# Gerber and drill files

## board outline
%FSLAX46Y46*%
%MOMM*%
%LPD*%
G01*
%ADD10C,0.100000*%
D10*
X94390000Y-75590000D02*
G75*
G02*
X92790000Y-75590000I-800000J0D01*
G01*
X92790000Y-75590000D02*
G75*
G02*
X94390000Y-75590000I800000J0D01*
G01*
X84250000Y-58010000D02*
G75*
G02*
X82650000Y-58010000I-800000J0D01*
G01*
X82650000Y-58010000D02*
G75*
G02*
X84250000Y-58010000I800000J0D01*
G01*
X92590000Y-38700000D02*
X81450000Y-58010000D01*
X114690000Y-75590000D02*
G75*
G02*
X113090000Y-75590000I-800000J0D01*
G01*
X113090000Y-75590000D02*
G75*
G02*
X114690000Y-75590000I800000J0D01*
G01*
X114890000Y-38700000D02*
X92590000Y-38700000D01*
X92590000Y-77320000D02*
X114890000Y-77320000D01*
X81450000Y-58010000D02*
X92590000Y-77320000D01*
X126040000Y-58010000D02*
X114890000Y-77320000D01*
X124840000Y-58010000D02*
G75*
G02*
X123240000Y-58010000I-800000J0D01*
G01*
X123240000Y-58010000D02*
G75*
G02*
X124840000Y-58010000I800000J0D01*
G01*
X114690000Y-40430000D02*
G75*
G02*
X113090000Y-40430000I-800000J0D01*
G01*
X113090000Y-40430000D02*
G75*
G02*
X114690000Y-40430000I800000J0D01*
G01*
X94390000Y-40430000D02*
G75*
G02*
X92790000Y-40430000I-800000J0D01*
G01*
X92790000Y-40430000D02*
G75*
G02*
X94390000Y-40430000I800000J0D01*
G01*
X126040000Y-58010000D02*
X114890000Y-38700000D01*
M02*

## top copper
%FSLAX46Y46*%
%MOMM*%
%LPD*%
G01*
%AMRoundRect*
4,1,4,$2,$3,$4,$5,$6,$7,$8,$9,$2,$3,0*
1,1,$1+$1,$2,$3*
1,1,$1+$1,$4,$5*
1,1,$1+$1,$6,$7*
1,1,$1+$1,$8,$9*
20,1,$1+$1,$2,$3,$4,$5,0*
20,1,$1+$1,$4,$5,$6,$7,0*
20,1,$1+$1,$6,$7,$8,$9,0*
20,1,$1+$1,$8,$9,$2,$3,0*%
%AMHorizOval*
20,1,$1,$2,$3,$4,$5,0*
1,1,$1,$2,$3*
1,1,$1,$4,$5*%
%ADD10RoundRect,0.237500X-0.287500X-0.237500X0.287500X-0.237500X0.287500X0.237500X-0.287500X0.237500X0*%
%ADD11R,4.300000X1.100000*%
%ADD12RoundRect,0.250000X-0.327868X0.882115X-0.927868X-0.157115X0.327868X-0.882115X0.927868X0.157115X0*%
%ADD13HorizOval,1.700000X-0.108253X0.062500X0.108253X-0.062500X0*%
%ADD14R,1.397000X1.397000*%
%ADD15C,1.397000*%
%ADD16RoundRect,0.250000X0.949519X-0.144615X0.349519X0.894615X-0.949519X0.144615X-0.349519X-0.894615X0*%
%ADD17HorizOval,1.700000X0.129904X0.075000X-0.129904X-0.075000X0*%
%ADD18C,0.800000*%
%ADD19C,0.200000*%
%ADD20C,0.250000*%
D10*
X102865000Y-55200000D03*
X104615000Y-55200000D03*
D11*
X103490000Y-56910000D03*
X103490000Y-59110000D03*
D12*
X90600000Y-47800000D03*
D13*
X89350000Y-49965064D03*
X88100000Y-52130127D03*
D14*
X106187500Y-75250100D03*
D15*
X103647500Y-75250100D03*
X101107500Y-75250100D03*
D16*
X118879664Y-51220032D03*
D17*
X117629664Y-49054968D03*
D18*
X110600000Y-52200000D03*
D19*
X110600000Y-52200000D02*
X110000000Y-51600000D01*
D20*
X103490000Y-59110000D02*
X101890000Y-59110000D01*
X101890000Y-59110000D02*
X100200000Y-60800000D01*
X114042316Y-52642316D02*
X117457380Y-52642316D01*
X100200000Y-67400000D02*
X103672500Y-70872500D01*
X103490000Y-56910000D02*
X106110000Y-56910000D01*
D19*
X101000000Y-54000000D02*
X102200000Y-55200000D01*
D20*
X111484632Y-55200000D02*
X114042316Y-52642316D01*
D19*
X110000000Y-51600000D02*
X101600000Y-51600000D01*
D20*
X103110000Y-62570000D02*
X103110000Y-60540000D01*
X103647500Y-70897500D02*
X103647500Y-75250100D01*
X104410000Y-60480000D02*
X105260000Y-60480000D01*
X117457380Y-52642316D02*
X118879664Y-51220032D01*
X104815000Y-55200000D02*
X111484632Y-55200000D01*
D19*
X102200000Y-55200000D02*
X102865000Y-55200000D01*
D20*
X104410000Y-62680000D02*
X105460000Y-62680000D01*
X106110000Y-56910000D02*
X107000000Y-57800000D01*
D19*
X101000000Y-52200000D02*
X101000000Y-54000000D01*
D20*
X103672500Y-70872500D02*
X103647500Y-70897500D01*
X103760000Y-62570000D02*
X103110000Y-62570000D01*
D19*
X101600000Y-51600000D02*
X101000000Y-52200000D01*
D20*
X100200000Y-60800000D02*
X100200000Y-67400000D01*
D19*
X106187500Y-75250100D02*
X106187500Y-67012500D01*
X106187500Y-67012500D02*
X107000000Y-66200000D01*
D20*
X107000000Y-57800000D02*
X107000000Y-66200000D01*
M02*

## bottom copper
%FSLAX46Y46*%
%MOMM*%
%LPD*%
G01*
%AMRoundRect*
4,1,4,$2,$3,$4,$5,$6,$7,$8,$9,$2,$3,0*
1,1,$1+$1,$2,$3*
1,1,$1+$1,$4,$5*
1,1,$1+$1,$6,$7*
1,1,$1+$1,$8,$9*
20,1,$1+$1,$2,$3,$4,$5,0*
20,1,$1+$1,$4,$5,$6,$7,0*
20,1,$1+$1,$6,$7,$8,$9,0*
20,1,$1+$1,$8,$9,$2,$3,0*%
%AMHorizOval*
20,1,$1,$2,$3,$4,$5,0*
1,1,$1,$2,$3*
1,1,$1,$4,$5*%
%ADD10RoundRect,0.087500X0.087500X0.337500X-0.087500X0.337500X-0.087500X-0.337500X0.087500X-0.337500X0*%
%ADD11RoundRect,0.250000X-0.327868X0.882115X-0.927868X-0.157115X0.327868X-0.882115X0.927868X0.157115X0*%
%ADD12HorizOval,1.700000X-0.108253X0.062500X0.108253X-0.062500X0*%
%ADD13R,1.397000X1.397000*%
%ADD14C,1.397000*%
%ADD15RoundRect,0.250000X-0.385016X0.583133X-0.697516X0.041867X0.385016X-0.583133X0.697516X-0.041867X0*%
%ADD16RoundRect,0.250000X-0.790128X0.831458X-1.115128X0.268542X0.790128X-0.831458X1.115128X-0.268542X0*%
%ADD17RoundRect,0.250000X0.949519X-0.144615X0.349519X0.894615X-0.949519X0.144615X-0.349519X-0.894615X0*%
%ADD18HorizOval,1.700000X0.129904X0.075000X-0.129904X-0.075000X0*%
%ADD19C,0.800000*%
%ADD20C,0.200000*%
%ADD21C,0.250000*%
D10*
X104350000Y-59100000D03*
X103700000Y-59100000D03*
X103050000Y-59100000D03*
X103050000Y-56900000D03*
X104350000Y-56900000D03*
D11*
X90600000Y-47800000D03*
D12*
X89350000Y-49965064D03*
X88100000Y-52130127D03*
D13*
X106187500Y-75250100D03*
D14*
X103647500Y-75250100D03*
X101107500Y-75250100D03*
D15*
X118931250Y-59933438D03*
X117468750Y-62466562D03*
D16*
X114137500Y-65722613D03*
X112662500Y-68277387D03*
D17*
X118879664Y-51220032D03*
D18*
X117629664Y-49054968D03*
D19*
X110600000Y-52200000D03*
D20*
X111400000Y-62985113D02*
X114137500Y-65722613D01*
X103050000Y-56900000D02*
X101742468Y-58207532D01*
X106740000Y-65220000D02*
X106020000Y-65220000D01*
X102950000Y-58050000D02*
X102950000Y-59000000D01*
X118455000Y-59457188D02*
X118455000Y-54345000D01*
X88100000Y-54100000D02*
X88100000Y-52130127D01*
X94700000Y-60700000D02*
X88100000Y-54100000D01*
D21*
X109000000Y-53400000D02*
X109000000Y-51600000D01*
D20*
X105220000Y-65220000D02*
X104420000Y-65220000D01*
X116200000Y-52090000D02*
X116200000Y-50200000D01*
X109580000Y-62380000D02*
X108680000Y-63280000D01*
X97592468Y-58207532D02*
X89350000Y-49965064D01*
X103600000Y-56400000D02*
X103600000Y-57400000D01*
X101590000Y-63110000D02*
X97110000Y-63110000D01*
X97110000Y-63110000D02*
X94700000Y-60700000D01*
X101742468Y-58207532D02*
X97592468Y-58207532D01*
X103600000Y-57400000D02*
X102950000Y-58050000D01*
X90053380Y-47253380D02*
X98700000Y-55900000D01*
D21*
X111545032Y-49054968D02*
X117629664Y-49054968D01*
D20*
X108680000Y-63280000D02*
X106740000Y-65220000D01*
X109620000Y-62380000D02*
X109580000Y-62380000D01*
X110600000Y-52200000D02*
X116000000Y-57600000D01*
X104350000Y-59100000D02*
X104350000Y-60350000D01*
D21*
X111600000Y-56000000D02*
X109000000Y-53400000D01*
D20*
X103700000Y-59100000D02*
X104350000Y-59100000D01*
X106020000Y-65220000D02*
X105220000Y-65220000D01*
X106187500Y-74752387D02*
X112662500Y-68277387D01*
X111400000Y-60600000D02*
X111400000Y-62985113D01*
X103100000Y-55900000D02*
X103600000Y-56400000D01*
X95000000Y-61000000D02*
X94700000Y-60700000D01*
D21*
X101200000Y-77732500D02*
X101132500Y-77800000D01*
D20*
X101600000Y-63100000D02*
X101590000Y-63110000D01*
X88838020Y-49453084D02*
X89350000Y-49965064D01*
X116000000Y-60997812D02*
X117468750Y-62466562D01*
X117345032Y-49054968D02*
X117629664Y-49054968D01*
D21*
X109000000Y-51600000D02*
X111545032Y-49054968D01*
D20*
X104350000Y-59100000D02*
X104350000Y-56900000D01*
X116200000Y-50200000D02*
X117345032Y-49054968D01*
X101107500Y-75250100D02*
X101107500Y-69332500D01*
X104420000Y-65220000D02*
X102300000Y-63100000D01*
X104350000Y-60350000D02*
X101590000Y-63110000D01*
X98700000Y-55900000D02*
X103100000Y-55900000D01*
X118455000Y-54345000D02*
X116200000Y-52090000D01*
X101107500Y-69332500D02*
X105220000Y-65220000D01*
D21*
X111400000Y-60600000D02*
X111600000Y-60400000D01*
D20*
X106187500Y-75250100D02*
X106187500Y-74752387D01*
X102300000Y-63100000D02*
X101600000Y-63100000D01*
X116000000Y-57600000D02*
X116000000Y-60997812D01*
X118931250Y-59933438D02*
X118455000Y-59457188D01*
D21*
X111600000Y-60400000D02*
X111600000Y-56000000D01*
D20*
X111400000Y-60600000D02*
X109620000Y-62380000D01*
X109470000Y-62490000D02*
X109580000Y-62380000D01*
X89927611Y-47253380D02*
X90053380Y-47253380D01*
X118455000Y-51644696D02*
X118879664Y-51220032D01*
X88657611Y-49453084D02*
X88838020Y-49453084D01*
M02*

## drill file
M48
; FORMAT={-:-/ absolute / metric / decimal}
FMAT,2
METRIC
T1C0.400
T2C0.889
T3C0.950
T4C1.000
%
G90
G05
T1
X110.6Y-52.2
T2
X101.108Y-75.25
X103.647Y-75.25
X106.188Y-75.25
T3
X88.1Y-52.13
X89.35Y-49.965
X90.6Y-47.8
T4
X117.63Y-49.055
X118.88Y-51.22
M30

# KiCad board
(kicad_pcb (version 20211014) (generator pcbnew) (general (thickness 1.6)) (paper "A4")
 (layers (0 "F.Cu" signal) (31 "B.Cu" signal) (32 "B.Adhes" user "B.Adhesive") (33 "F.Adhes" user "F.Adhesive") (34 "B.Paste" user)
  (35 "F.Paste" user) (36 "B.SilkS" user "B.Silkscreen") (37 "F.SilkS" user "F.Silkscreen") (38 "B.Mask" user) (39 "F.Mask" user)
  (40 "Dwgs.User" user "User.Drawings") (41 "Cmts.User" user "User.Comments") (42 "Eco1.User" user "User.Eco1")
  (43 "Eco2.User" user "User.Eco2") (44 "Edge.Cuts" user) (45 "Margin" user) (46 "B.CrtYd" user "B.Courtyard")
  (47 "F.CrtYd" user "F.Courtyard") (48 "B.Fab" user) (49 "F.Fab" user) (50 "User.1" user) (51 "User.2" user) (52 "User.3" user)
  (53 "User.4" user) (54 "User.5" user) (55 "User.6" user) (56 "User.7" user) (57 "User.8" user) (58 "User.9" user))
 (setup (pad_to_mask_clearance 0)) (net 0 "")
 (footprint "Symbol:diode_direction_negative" (layer "F.Cu") (at 103.8 52.65)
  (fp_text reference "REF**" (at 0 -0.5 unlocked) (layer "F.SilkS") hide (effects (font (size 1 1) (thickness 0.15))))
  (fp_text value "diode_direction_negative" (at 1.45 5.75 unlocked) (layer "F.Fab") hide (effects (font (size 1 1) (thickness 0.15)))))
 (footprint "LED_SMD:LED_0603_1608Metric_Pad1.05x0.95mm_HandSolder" (layer "F.Cu") (at 103.74 55.2)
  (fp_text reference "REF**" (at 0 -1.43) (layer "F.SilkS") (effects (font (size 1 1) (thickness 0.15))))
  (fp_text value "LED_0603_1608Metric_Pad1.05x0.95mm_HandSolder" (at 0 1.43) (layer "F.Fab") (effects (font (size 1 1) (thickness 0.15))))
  (pad "1" smd roundrect (at -0.875 0) (size 1.05 0.95) (layers "F.Cu" "F.Paste" "F.Mask") (roundrect_rratio 0.25))
  (pad "2" smd roundrect (at 0.875 0) (size 1.05 0.95) (layers "F.Cu" "F.Paste" "F.Mask") (roundrect_rratio 0.25)))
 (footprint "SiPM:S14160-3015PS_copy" (layer "F.Cu") (at 103.74 58.01)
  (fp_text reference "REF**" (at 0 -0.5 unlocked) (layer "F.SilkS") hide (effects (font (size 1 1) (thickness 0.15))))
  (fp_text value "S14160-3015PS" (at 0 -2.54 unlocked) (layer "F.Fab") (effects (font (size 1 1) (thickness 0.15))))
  (pad "1" smd rect (at -0.25 -1.1) (size 4.3 1.1) (layers "F.Cu" "F.Paste" "F.Mask"))
  (pad "2" smd rect (at -0.25 1.1) (size 4.3 1.1) (layers "F.Cu" "F.Paste" "F.Mask")))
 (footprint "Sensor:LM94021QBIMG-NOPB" (layer "B.Cu") (at 103.7 58 180)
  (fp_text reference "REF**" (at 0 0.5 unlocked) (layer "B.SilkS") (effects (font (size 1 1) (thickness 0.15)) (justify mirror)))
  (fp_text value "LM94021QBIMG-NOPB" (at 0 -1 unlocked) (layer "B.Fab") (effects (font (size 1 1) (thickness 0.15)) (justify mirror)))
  (pad "1" smd roundrect (at -0.65 -1.1 180) (size 0.35 0.85) (layers "B.Cu" "B.Paste" "B.Mask") (roundrect_rratio 0.25))
  (pad "2" smd roundrect (at 0 -1.1 180) (size 0.35 0.85) (layers "B.Cu" "B.Paste" "B.Mask") (roundrect_rratio 0.25))
  (pad "3" smd roundrect (at 0.65 -1.1 180) (size 0.35 0.85) (layers "B.Cu" "B.Paste" "B.Mask") (roundrect_rratio 0.25))
  (pad "4" smd roundrect (at 0.65 1.1 180) (size 0.35 0.85) (layers "B.Cu" "B.Paste" "B.Mask") (roundrect_rratio 0.25))
  (pad "5" smd roundrect (at -0.65 1.1 180) (size 0.35 0.85) (layers "B.Cu" "B.Paste" "B.Mask") (roundrect_rratio 0.25)))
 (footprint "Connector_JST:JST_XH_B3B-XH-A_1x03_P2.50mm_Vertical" (layer "B.Cu") (at 90.6 47.8 -120)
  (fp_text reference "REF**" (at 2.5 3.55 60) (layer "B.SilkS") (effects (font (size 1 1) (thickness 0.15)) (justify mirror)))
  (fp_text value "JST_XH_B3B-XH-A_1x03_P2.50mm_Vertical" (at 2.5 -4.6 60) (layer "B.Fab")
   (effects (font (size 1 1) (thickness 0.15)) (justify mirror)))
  (pad "1" thru_hole roundrect (at 0 0 240) (size 1.7 1.95) (drill 0.95) (layers *.Cu *.Mask) (roundrect_rratio 0.1470588235))
  (pad "2" thru_hole oval (at 2.5 0 240) (size 1.7 1.95) (drill 0.95) (layers *.Cu *.Mask))
  (pad "3" thru_hole oval (at 5 0 240) (size 1.7 1.95) (drill 0.95) (layers *.Cu *.Mask)))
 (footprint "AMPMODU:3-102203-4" (layer "B.Cu") (at 106.1875 75.2501 180)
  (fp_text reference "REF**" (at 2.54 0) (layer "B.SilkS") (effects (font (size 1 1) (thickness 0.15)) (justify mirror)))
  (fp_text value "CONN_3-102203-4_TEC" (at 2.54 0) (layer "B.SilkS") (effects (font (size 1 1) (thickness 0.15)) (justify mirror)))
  (pad "1" thru_hole rect locked (at 0 0 180) (size 1.397 1.397) (drill 0.889) (layers *.Cu *.Mask))
  (pad "2" thru_hole circle locked (at 2.54 0 180) (size 1.397 1.397) (drill 0.889) (layers *.Cu *.Mask))
  (pad "3" thru_hole circle locked (at 5.08 0 180) (size 1.397 1.397) (drill 0.889) (layers *.Cu *.Mask)))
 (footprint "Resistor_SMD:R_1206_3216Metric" (layer "B.Cu") (at 118.2 61.2 -120)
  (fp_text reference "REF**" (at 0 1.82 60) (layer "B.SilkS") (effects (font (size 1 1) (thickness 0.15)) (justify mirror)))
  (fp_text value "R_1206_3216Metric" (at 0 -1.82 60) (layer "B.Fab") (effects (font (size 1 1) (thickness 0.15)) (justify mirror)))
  (pad "1" smd roundrect (at -1.4625 0 240) (size 1.125 1.75) (layers "B.Cu" "B.Paste" "B.Mask") (roundrect_rratio 0.222222))
  (pad "2" smd roundrect (at 1.4625 0 240) (size 1.125 1.75) (layers "B.Cu" "B.Paste" "B.Mask") (roundrect_rratio 0.222222)))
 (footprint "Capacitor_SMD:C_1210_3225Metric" (layer "B.Cu") (at 113.4 67 -120)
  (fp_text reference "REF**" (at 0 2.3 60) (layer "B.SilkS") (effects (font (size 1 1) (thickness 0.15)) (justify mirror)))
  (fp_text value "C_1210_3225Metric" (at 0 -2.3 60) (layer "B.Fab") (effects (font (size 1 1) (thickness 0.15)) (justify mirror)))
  (pad "1" smd roundrect (at -1.475 0 240) (size 1.15 2.7) (layers "B.Cu" "B.Paste" "B.Mask") (roundrect_rratio 0.2173913043))
  (pad "2" smd roundrect (at 1.475 0 240) (size 1.15 2.7) (layers "B.Cu" "B.Paste" "B.Mask") (roundrect_rratio 0.2173913043)))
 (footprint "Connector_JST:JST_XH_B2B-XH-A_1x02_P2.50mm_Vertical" (layer "B.Cu") (at 118.879664 51.220032 120)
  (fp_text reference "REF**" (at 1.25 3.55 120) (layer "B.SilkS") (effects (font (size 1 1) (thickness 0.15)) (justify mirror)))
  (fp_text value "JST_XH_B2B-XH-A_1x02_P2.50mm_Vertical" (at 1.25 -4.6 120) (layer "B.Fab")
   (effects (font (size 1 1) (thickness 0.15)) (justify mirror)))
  (pad "1" thru_hole roundrect (at 0 0 120) (size 1.7 2) (drill 1) (layers *.Cu *.Mask) (roundrect_rratio 0.1470588235))
  (pad "2" thru_hole oval (at 2.5 0 120) (size 1.7 2) (drill 1) (layers *.Cu *.Mask)))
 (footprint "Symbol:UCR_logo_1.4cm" (layer "B.Cu") (at 104.4 43 180)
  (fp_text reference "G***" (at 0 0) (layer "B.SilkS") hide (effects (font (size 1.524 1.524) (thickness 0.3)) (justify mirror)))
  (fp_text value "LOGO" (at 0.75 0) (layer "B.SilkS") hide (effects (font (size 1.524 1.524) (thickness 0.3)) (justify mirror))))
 (gr_circle (center 93.59 75.59) (end 94.39 75.59) (layer "Edge.Cuts") (width 0.1) (fill none))
 (gr_circle (center 83.45 58.01) (end 84.25 58.01) (layer "Edge.Cuts") (width 0.1) (fill none))
 (gr_line (start 92.59 38.7) (end 81.45 58.01) (layer "Edge.Cuts") (width 0.1))
 (gr_circle (center 113.89 75.59) (end 114.69 75.59) (layer "Edge.Cuts") (width 0.1) (fill none))
 (gr_line (start 114.89 38.7) (end 92.59 38.7) (layer "Edge.Cuts") (width 0.1))
 (gr_line (start 92.59 77.32) (end 114.89 77.32) (layer "Edge.Cuts") (width 0.1))
 (gr_line (start 81.45 58.01) (end 92.59 77.32) (layer "Edge.Cuts") (width 0.1))
 (gr_line (start 126.04 58.01) (end 114.89 77.32) (layer "Edge.Cuts") (width 0.1))
 (gr_circle (center 124.04 58.01) (end 124.84 58.01) (layer "Edge.Cuts") (width 0.1) (fill none))
 (gr_circle (center 113.89 40.43) (end 114.69 40.43) (layer "Edge.Cuts") (width 0.1) (fill none))
 (gr_circle (center 93.59 40.43) (end 94.39 40.43) (layer "Edge.Cuts") (width 0.1) (fill none))
 (gr_line (start 126.04 58.01) (end 114.89 38.7) (layer "Edge.Cuts") (width 0.1))
 (segment (start 110.6 52.2) (end 110 51.6) (width 0.2) (layer "F.Cu") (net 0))
 (segment (start 103.49 59.11) (end 101.89 59.11) (width 0.25) (layer "F.Cu") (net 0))
 (segment (start 101.89 59.11) (end 100.2 60.8) (width 0.25) (layer "F.Cu") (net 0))
 (segment (start 114.042316 52.642316) (end 117.45738 52.642316) (width 0.25) (layer "F.Cu") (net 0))
 (segment (start 100.2 67.4) (end 103.6725 70.8725) (width 0.25) (layer "F.Cu") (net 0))
 (segment (start 103.49 56.91) (end 106.11 56.91) (width 0.25) (layer "F.Cu") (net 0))
 (segment (start 101 54) (end 102.2 55.2) (width 0.2) (layer "F.Cu") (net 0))
 (segment (start 111.484632 55.2) (end 114.042316 52.642316) (width 0.25) (layer "F.Cu") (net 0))
 (segment (start 110 51.6) (end 101.6 51.6) (width 0.2) (layer "F.Cu") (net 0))
 (segment (start 103.11 62.57) (end 103.11 60.54) (width 0.25) (layer "F.Cu") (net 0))
 (segment (start 103.6475 70.8975) (end 103.6475 75.2501) (width 0.25) (layer "F.Cu") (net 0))
 (segment (start 104.41 60.48) (end 105.26 60.48) (width 0.25) (layer "F.Cu") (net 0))
 (segment (start 117.45738 52.642316) (end 118.879664 51.220032) (width 0.25) (layer "F.Cu") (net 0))
 (segment (start 104.815 55.2) (end 111.484632 55.2) (width 0.25) (layer "F.Cu") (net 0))
 (segment (start 102.2 55.2) (end 102.865 55.2) (width 0.2) (layer "F.Cu") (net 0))
 (segment (start 104.41 62.68) (end 105.46 62.68) (width 0.25) (layer "F.Cu") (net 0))
 (segment (start 106.11 56.91) (end 107 57.8) (width 0.25) (layer "F.Cu") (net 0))
 (segment (start 101 52.2) (end 101 54) (width 0.2) (layer "F.Cu") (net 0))
 (segment (start 103.6725 70.8725) (end 103.6475 70.8975) (width 0.25) (layer "F.Cu") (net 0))
 (segment (start 103.76 62.57) (end 103.11 62.57) (width 0.25) (layer "F.Cu") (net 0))
 (segment (start 101.6 51.6) (end 101 52.2) (width 0.2) (layer "F.Cu") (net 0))
 (segment (start 100.2 60.8) (end 100.2 67.4) (width 0.25) (layer "F.Cu") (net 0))
 (segment (start 106.1875 75.2501) (end 106.1875 67.0125) (width 0.2) (layer "F.Cu") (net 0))
 (segment (start 106.1875 67.0125) (end 107 66.2) (width 0.2) (layer "F.Cu") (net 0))
 (segment (start 107 57.8) (end 107 66.2) (width 0.25) (layer "F.Cu") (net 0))
 (via (at 110.6 52.2) (size 0.8) (drill 0.4) (layers "F.Cu" "B.Cu") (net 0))
 (segment (start 111.4 62.985113) (end 114.1375 65.722613) (width 0.2) (layer "B.Cu") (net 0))
 (segment (start 103.05 56.9) (end 101.742468 58.207532) (width 0.2) (layer "B.Cu") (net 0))
 (segment (start 106.74 65.22) (end 106.02 65.22) (width 0.2) (layer "B.Cu") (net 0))
 (segment (start 102.95 58.05) (end 102.95 59) (width 0.2) (layer "B.Cu") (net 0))
 (segment (start 118.455 59.457188) (end 118.455 54.345) (width 0.2) (layer "B.Cu") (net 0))
 (segment (start 88.1 54.1) (end 88.1 52.130127) (width 0.2) (layer "B.Cu") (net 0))
 (segment (start 94.7 60.7) (end 88.1 54.1) (width 0.2) (layer "B.Cu") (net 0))
 (segment (start 109 53.4) (end 109 51.6) (width 0.25) (layer "B.Cu") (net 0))
 (segment (start 105.22 65.22) (end 104.42 65.22) (width 0.2) (layer "B.Cu") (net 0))
 (segment (start 116.2 52.09) (end 116.2 50.2) (width 0.2) (layer "B.Cu") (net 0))
 (segment (start 109.58 62.38) (end 108.68 63.28) (width 0.2) (layer "B.Cu") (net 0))
 (segment (start 97.592468 58.207532) (end 89.35 49.965064) (width 0.2) (layer "B.Cu") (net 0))
 (segment (start 103.6 56.4) (end 103.6 57.4) (width 0.2) (layer "B.Cu") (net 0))
 (segment (start 101.59 63.11) (end 97.11 63.11) (width 0.2) (layer "B.Cu") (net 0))
 (segment (start 97.11 63.11) (end 94.7 60.7) (width 0.2) (layer "B.Cu") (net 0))
 (segment (start 101.742468 58.207532) (end 97.592468 58.207532) (width 0.2) (layer "B.Cu") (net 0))
 (segment (start 103.6 57.4) (end 102.95 58.05) (width 0.2) (layer "B.Cu") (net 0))
 (segment (start 90.05338 47.25338) (end 98.7 55.9) (width 0.2) (layer "B.Cu") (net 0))
 (segment (start 111.545032 49.054968) (end 117.629664 49.054968) (width 0.25) (layer "B.Cu") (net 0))
 (segment (start 108.68 63.28) (end 106.74 65.22) (width 0.2) (layer "B.Cu") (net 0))
 (segment (start 109.62 62.38) (end 109.58 62.38) (width 0.2) (layer "B.Cu") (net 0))
 (segment (start 110.6 52.2) (end 116 57.6) (width 0.2) (layer "B.Cu") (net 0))
 (segment (start 104.35 59.1) (end 104.35 60.35) (width 0.2) (layer "B.Cu") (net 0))
 (segment (start 111.6 56) (end 109 53.4) (width 0.25) (layer "B.Cu") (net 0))
 (segment (start 103.7 59.1) (end 104.35 59.1) (width 0.2) (layer "B.Cu") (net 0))
 (segment (start 106.02 65.22) (end 105.22 65.22) (width 0.2) (layer "B.Cu") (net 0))
 (segment (start 106.1875 74.752387) (end 112.6625 68.277387) (width 0.2) (layer "B.Cu") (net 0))
 (segment (start 111.4 60.6) (end 111.4 62.985113) (width 0.2) (layer "B.Cu") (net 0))
 (segment (start 103.1 55.9) (end 103.6 56.4) (width 0.2) (layer "B.Cu") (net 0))
 (segment (start 95 61) (end 94.7 60.7) (width 0.2) (layer "B.Cu") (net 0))
 (segment (start 101.2 77.7325) (end 101.1325 77.8) (width 0.25) (layer "B.Cu") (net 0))
 (segment (start 101.6 63.1) (end 101.59 63.11) (width 0.2) (layer "B.Cu") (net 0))
 (segment (start 88.83802 49.453084) (end 89.35 49.965064) (width 0.2) (layer "B.Cu") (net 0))
 (segment (start 116 60.997812) (end 117.46875 62.466562) (width 0.2) (layer "B.Cu") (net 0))
 (segment (start 117.345032 49.054968) (end 117.629664 49.054968) (width 0.2) (layer "B.Cu") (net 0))
 (segment (start 109 51.6) (end 111.545032 49.054968) (width 0.25) (layer "B.Cu") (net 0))
 (segment (start 104.35 59.1) (end 104.35 56.9) (width 0.2) (layer "B.Cu") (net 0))
 (segment (start 116.2 50.2) (end 117.345032 49.054968) (width 0.2) (layer "B.Cu") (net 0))
 (segment (start 101.1075 75.2501) (end 101.1075 69.3325) (width 0.2) (layer "B.Cu") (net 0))
 (segment (start 104.42 65.22) (end 102.3 63.1) (width 0.2) (layer "B.Cu") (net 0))
 (segment (start 104.35 60.35) (end 101.59 63.11) (width 0.2) (layer "B.Cu") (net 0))
 (segment (start 98.7 55.9) (end 103.1 55.9) (width 0.2) (layer "B.Cu") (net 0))
 (segment (start 118.455 54.345) (end 116.2 52.09) (width 0.2) (layer "B.Cu") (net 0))
 (segment (start 101.1075 69.3325) (end 105.22 65.22) (width 0.2) (layer "B.Cu") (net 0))
 (segment (start 111.4 60.6) (end 111.6 60.4) (width 0.25) (layer "B.Cu") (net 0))
 (segment (start 106.1875 75.2501) (end 106.1875 74.752387) (width 0.2) (layer "B.Cu") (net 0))
 (segment (start 102.3 63.1) (end 101.6 63.1) (width 0.2) (layer "B.Cu") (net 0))
 (segment (start 116 57.6) (end 116 60.997812) (width 0.2) (layer "B.Cu") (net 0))
 (segment (start 118.93125 59.933438) (end 118.455 59.457188) (width 0.2) (layer "B.Cu") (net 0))
 (segment (start 111.6 60.4) (end 111.6 56) (width 0.25) (layer "B.Cu") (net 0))
 (segment (start 111.4 60.6) (end 109.62 62.38) (width 0.2) (layer "B.Cu") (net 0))
 (segment (start 109.47 62.49) (end 109.58 62.38) (width 0.2) (layer "B.Cu") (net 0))
 (segment (start 89.927611 47.25338) (end 90.05338 47.25338) (width 0.2) (layer "B.Cu") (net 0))
 (segment (start 118.455 51.644696) (end 118.879664 51.220032) (width 0.2) (layer "B.Cu") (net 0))
 (segment (start 88.657611 49.453084) (end 88.83802 49.453084) (width 0.2) (layer "B.Cu") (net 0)))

